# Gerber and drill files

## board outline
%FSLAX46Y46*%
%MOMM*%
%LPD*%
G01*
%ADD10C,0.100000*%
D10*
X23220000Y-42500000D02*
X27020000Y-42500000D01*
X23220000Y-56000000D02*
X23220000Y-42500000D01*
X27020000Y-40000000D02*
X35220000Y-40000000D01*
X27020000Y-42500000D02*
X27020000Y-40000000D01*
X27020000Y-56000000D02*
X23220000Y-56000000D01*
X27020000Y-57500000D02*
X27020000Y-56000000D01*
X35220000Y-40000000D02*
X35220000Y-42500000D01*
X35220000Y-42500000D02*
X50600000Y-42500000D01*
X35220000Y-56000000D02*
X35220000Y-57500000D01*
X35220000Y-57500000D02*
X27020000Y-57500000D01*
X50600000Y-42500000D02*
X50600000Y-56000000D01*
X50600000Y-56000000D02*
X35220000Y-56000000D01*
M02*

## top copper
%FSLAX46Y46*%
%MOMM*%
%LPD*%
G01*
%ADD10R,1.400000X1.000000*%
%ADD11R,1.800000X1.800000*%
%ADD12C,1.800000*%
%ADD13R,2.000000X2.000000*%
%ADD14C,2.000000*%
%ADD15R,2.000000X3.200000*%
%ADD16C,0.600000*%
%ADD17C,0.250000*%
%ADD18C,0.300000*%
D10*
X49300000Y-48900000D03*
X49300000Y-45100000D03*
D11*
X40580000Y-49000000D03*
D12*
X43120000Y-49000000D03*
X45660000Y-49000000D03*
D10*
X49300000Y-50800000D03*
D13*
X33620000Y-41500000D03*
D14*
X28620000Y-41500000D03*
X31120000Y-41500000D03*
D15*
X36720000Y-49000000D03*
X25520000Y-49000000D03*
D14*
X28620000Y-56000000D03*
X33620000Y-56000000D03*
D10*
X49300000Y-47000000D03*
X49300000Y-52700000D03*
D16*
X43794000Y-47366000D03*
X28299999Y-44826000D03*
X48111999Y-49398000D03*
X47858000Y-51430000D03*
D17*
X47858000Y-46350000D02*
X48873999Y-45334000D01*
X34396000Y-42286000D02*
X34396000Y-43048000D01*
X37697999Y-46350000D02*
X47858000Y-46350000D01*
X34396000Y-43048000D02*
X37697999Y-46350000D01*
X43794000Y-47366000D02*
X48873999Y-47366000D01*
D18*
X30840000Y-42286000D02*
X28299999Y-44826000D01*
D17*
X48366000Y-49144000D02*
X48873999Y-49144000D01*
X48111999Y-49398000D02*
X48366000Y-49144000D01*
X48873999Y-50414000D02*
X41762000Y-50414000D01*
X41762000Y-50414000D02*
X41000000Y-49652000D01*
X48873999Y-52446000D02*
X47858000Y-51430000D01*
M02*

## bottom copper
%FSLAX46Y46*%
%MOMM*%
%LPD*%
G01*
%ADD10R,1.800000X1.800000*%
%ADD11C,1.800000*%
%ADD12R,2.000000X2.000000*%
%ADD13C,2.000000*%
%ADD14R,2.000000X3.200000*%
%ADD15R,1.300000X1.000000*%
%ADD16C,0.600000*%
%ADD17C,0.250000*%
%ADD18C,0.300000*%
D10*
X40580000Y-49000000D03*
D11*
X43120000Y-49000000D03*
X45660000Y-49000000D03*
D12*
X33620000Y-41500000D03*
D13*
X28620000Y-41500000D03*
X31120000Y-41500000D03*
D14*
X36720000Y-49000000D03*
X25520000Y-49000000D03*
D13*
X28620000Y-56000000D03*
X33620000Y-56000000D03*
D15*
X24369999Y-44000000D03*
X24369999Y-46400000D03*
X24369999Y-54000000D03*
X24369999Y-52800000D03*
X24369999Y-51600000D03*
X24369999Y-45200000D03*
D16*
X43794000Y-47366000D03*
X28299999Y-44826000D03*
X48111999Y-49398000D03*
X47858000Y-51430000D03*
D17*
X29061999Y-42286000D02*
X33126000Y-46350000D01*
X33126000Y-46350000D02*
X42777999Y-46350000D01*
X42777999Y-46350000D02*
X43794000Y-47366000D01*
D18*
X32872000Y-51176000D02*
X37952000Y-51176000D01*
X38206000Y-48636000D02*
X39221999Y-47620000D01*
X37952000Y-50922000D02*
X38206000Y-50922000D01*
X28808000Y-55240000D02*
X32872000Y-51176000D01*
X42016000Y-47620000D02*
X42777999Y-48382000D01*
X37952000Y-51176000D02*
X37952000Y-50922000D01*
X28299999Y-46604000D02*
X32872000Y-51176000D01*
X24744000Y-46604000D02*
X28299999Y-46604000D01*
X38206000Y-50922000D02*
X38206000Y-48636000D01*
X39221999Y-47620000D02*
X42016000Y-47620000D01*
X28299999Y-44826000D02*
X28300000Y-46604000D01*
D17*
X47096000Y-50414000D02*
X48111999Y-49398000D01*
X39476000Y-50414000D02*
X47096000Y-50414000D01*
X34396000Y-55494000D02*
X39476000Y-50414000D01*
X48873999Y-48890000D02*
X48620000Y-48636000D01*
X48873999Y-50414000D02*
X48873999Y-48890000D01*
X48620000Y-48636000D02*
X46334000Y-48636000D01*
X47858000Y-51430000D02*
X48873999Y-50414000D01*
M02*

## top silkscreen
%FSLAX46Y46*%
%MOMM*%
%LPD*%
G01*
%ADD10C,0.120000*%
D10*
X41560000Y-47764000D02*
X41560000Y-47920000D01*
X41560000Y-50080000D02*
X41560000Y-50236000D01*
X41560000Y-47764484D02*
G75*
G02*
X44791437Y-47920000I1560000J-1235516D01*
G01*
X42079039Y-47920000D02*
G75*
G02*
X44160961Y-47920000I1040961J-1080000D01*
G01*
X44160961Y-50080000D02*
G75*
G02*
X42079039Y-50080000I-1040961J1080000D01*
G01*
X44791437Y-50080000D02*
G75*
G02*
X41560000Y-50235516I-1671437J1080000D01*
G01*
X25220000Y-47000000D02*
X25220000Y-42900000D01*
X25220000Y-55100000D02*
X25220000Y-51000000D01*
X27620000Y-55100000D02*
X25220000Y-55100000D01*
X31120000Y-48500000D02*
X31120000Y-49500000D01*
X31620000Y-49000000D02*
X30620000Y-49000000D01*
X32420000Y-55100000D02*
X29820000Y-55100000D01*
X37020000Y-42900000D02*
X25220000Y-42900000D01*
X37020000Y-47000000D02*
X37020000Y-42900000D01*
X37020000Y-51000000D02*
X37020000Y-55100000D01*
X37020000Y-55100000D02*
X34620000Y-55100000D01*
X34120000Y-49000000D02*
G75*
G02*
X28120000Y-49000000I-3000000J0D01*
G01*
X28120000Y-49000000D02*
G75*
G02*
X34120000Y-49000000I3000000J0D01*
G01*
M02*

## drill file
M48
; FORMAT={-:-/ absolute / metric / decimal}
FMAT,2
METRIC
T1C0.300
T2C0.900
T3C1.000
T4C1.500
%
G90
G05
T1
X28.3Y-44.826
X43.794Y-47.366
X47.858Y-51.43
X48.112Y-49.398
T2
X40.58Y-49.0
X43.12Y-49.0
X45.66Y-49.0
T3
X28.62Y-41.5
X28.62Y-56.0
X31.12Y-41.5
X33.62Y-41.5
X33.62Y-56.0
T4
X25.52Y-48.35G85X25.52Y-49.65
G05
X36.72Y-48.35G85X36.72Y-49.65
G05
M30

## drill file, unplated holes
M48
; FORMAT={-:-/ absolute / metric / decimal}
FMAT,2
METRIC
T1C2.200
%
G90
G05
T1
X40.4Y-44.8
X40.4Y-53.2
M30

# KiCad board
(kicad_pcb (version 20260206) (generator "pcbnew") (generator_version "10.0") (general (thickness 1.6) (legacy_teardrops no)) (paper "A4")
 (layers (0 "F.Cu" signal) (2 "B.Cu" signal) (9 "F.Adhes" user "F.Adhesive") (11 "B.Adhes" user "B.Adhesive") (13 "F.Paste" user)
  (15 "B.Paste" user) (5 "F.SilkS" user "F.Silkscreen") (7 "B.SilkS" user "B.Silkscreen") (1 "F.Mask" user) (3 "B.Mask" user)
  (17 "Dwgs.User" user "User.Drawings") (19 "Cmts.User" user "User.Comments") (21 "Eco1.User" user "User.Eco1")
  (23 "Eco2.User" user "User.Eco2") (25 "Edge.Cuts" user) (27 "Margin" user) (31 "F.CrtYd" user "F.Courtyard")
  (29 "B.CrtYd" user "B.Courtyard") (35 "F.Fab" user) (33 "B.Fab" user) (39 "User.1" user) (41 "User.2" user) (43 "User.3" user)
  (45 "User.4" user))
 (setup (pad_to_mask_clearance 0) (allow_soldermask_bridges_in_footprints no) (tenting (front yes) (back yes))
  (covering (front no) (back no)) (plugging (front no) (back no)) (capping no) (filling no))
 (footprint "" (layer "F.Cu") (at 49.3 48.9)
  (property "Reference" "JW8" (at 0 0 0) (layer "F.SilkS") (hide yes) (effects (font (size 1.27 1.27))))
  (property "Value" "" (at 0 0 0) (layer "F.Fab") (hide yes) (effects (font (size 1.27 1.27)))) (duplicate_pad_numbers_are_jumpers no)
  (pad "1" smd rect (at 0 0) (size 1.4 1) (layers "F.Cu" "F.Mask" "F.Paste") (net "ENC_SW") (thermal_bridge_angle 45)))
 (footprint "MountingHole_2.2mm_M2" (layer "F.Cu") (at 40.4 44.8)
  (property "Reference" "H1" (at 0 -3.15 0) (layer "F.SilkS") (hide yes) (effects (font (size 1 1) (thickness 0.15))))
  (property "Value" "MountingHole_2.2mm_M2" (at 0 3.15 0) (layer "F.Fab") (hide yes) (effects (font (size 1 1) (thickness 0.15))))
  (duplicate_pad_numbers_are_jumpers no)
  (pad "" np_thru_hole circle (at 0 0) (size 2.2 2.2) (drill 2.2) (layers "*.Cu" "*.Mask")))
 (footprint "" (layer "F.Cu") (at 49.3 45.1)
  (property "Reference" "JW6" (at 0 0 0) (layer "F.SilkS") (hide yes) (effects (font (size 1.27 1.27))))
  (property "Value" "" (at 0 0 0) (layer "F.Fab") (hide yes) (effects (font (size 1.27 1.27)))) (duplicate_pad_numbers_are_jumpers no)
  (pad "1" smd rect (at 0 0) (size 1.4 1) (layers "F.Cu" "F.Mask" "F.Paste") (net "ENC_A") (thermal_bridge_angle 45)))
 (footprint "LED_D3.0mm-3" (layer "F.Cu") (at 40.58 49)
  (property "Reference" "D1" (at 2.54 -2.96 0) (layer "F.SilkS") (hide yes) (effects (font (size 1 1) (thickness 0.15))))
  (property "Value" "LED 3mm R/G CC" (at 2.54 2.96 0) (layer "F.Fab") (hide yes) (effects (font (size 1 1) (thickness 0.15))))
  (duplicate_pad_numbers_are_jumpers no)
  (fp_line (start 0.98 -1.236) (end 0.98 -1.08) (stroke (width 0.12) (type solid)) (layer "F.SilkS"))
  (fp_line (start 0.98 1.08) (end 0.98 1.236) (stroke (width 0.12) (type solid)) (layer "F.SilkS"))
  (fp_arc (start 0.98 -1.235516) (mid 2.63566 -1.987699) (end 4.211437 -1.08) (stroke (width 0.12) (type solid)) (layer "F.SilkS"))
  (fp_arc (start 1.499039 -1.08) (mid 2.54 -1.5) (end 3.580961 -1.08) (stroke (width 0.12) (type solid)) (layer "F.SilkS"))
  (fp_arc (start 3.580961 1.08) (mid 2.54 1.5) (end 1.499039 1.08) (stroke (width 0.12) (type solid)) (layer "F.SilkS"))
  (fp_arc (start 4.211437 1.08) (mid 2.63566 1.987699) (end 0.98 1.235516) (stroke (width 0.12) (type solid)) (layer "F.SilkS"))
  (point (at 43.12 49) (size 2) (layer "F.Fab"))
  (pad "1" thru_hole rect (at 0 0) (size 1.8 1.8) (drill 0.9) (layers "*.Cu" "*.Mask") (remove_unused_layers no) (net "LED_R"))
  (pad "2" thru_hole circle (at 2.54 0) (size 1.8 1.8) (drill 0.9) (layers "*.Cu" "*.Mask") (remove_unused_layers no) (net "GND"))
  (pad "3" thru_hole circle (at 5.08 0) (size 1.8 1.8) (drill 0.9) (layers "*.Cu" "*.Mask") (remove_unused_layers no) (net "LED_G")))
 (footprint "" (layer "F.Cu") (at 49.3 50.8)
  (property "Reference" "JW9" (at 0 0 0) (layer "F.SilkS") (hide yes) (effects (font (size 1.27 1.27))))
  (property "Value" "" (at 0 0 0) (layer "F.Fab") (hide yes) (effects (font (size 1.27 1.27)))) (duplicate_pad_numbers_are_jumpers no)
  (pad "1" smd rect (at 0 0) (size 1.4 1) (layers "F.Cu" "F.Mask" "F.Paste") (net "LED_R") (thermal_bridge_angle 45)))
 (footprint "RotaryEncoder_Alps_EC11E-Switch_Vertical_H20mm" (layer "F.Cu") (at 33.62 41.5 -90)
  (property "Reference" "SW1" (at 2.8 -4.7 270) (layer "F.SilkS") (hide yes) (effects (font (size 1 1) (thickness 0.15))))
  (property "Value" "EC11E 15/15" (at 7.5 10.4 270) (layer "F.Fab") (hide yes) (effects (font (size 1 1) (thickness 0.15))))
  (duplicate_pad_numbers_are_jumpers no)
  (fp_line (start 5.5 8.4) (end 1.4 8.4) (stroke (width 0.12) (type solid)) (layer "F.SilkS"))
  (fp_line (start 13.6 8.4) (end 9.5 8.4) (stroke (width 0.12) (type solid)) (layer "F.SilkS"))
  (fp_line (start 13.6 6) (end 13.6 8.4) (stroke (width 0.12) (type solid)) (layer "F.SilkS"))
  (fp_line (start 7 2.5) (end 8 2.5) (stroke (width 0.12) (type solid)) (layer "F.SilkS"))
  (fp_line (start 7.5 2) (end 7.5 3) (stroke (width 0.12) (type solid)) (layer "F.SilkS"))
  (fp_line (start 13.6 1.2) (end 13.6 3.8) (stroke (width 0.12) (type solid)) (layer "F.SilkS"))
  (fp_line (start 1.4 -3.4) (end 1.4 8.4) (stroke (width 0.12) (type solid)) (layer "F.SilkS"))
  (fp_line (start 5.5 -3.4) (end 1.4 -3.4) (stroke (width 0.12) (type solid)) (layer "F.SilkS"))
  (fp_line (start 9.5 -3.4) (end 13.6 -3.4) (stroke (width 0.12) (type solid)) (layer "F.SilkS"))
  (fp_line (start 13.6 -3.4) (end 13.6 -1) (stroke (width 0.12) (type solid)) (layer "F.SilkS"))
  (fp_circle (center 7.5 2.5) (end 10.5 2.5) (stroke (width 0.12) (type solid)) (fill no) (layer "F.SilkS"))
  (pad "A" thru_hole rect (at 0 0 270) (size 2 2) (drill 1) (layers "*.Cu" "*.Mask") (remove_unused_layers no) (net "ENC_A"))
  (pad "B" thru_hole circle (at 0 5 270) (size 2 2) (drill 1) (layers "*.Cu" "*.Mask") (remove_unused_layers no) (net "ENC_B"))
  (pad "C" thru_hole circle (at 0 2.5 270) (size 2 2) (drill 1) (layers "*.Cu" "*.Mask") (remove_unused_layers no) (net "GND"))
  (pad "MP" thru_hole rect (at 7.5 -3.1 270) (size 3.2 2) (drill oval 2.8 1.5) (layers "*.Cu" "*.Mask") (remove_unused_layers no))
  (pad "MP" thru_hole rect (at 7.5 8.1 270) (size 3.2 2) (drill oval 2.8 1.5) (layers "*.Cu" "*.Mask") (remove_unused_layers no))
  (pad "S1" thru_hole circle (at 14.5 5 270) (size 2 2) (drill 1) (layers "*.Cu" "*.Mask") (remove_unused_layers no) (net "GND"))
  (pad "S2" thru_hole circle (at 14.5 0 270) (size 2 2) (drill 1) (layers "*.Cu" "*.Mask") (remove_unused_layers no) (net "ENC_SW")))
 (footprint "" (layer "F.Cu") (at 49.3 47)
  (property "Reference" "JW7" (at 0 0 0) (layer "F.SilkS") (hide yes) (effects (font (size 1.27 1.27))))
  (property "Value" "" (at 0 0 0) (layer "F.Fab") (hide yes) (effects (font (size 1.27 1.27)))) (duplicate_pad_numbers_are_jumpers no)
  (pad "1" smd rect (at 0 0) (size 1.4 1) (layers "F.Cu" "F.Mask" "F.Paste") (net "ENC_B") (thermal_bridge_angle 45)))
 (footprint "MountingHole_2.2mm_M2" (layer "F.Cu") (at 40.4 53.2)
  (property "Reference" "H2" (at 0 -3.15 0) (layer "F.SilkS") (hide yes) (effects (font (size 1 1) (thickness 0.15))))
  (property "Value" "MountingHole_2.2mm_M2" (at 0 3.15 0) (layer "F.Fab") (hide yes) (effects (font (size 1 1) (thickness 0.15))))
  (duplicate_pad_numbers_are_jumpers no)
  (pad "" np_thru_hole circle (at 0 0) (size 2.2 2.2) (drill 2.2) (layers "*.Cu" "*.Mask")))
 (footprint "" (layer "F.Cu") (at 49.3 52.7)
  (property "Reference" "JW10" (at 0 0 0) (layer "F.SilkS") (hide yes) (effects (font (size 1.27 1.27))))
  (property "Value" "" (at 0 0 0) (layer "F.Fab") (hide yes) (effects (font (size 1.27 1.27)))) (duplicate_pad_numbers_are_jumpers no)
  (pad "1" smd rect (at 0 0) (size 1.4 1) (layers "F.Cu" "F.Mask" "F.Paste") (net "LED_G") (thermal_bridge_angle 45)))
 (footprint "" (layer "B.Cu") (at 24.369999 44 180)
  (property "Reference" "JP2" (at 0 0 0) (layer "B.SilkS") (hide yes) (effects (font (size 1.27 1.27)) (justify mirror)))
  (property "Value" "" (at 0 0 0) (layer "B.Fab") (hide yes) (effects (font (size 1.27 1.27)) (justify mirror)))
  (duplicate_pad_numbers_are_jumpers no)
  (pad "1" smd rect (at 0 0 180) (size 1.3 1) (layers "B.Cu" "B.Mask" "B.Paste") (thermal_bridge_angle 45)))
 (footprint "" (layer "B.Cu") (at 24.369999 46.4 180)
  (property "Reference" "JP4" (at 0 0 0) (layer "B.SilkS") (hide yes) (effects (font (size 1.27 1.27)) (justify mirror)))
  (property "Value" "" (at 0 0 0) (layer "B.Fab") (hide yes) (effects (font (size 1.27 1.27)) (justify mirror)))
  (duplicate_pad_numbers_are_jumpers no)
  (pad "1" smd rect (at 0 0 180) (size 1.3 1) (layers "B.Cu" "B.Mask" "B.Paste") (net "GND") (thermal_bridge_angle 45)))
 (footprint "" (layer "B.Cu") (at 24.369999 54 180)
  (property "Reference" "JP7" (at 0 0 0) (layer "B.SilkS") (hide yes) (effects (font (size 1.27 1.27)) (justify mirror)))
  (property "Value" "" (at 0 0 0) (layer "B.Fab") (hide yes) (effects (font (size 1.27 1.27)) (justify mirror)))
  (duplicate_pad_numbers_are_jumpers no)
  (pad "1" smd rect (at 0 0 180) (size 1.3 1) (layers "B.Cu" "B.Mask" "B.Paste") (thermal_bridge_angle 45)))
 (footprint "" (layer "B.Cu") (at 24.369999 52.8 180)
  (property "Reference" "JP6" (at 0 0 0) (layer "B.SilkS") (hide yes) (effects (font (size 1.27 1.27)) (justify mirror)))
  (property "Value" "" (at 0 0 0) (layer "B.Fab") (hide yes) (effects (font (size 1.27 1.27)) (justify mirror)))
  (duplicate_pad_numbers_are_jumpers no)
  (pad "1" smd rect (at 0 0 180) (size 1.3 1) (layers "B.Cu" "B.Mask" "B.Paste") (thermal_bridge_angle 45)))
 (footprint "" (layer "B.Cu") (at 24.369999 51.6 180)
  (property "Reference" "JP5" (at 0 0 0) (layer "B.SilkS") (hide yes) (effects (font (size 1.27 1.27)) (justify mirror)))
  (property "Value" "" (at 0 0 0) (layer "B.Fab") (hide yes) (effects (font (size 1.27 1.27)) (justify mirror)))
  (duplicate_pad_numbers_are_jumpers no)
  (pad "1" smd rect (at 0 0 180) (size 1.3 1) (layers "B.Cu" "B.Mask" "B.Paste") (thermal_bridge_angle 45)))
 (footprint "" (layer "B.Cu") (at 24.369999 45.2 180)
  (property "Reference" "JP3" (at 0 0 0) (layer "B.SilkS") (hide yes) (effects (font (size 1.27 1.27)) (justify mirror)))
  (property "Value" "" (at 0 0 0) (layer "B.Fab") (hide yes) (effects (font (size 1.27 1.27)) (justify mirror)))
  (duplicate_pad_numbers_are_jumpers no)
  (pad "1" smd rect (at 0 0 180) (size 1.3 1) (layers "B.Cu" "B.Mask" "B.Paste") (thermal_bridge_angle 45)))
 (gr_line (start 23.22 42.5) (end 27.02 42.5) (stroke (width 0.1) (type default)) (layer "Edge.Cuts"))
 (gr_line (start 23.22 56) (end 23.22 42.5) (stroke (width 0.1) (type default)) (layer "Edge.Cuts"))
 (gr_line (start 27.02 40) (end 35.22 40) (stroke (width 0.1) (type default)) (layer "Edge.Cuts"))
 (gr_line (start 27.02 42.5) (end 27.02 40) (stroke (width 0.1) (type default)) (layer "Edge.Cuts"))
 (gr_line (start 27.02 56) (end 23.22 56) (stroke (width 0.1) (type default)) (layer "Edge.Cuts"))
 (gr_line (start 27.02 57.5) (end 27.02 56) (stroke (width 0.1) (type default)) (layer "Edge.Cuts"))
 (gr_line (start 35.22 40) (end 35.22 42.5) (stroke (width 0.1) (type default)) (layer "Edge.Cuts"))
 (gr_line (start 35.22 42.5) (end 50.6 42.5) (stroke (width 0.1) (type default)) (layer "Edge.Cuts"))
 (gr_line (start 35.22 56) (end 35.22 57.5) (stroke (width 0.1) (type default)) (layer "Edge.Cuts"))
 (gr_line (start 35.22 57.5) (end 27.02 57.5) (stroke (width 0.1) (type default)) (layer "Edge.Cuts"))
 (gr_line (start 50.6 42.5) (end 50.6 56) (stroke (width 0.1) (type default)) (layer "Edge.Cuts"))
 (gr_line (start 50.6 56) (end 35.22 56) (stroke (width 0.1) (type default)) (layer "Edge.Cuts"))
 (segment (start 47.858 46.35) (end 48.873999 45.334) (width 0.25) (layer "F.Cu") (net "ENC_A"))
 (segment (start 34.396 42.286) (end 34.396 43.048) (width 0.25) (layer "F.Cu") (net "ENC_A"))
 (segment (start 37.697999 46.35) (end 47.858 46.35) (width 0.25) (layer "F.Cu") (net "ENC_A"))
 (segment (start 34.396 43.048) (end 37.697999 46.35) (width 0.25) (layer "F.Cu") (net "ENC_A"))
 (segment (start 43.794 47.366) (end 48.873999 47.366) (width 0.25) (layer "F.Cu") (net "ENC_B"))
 (via (at 43.794 47.366) (size 0.6) (drill 0.3) (layers "F.Cu" "B.Cu") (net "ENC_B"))
 (segment (start 29.061999 42.286) (end 33.126 46.35) (width 0.25) (layer "B.Cu") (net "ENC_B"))
 (segment (start 33.126 46.35) (end 42.777999 46.35) (width 0.25) (layer "B.Cu") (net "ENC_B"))
 (segment (start 42.777999 46.35) (end 43.794 47.366) (width 0.25) (layer "B.Cu") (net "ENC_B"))
 (segment (start 30.84 42.286) (end 28.299999 44.826) (width 0.3) (layer "F.Cu") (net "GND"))
 (via (at 28.299999 44.826) (size 0.6) (drill 0.3) (layers "F.Cu" "B.Cu") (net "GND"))
 (segment (start 32.872 51.176) (end 37.952 51.176) (width 0.3) (layer "B.Cu") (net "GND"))
 (segment (start 38.206 48.636) (end 39.221999 47.62) (width 0.3) (layer "B.Cu") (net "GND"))
 (segment (start 37.952 50.922) (end 38.206 50.922) (width 0.3) (layer "B.Cu") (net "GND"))
 (segment (start 28.808 55.24) (end 32.872 51.176) (width 0.3) (layer "B.Cu") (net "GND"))
 (segment (start 42.016 47.62) (end 42.777999 48.382) (width 0.3) (layer "B.Cu") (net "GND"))
 (segment (start 37.952 51.176) (end 37.952 50.922) (width 0.3) (layer "B.Cu") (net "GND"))
 (segment (start 28.299999 46.604) (end 32.872 51.176) (width 0.3) (layer "B.Cu") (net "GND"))
 (segment (start 24.744 46.604) (end 28.299999 46.604) (width 0.3) (layer "B.Cu") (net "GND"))
 (segment (start 38.206 50.922) (end 38.206 48.636) (width 0.3) (layer "B.Cu") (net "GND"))
 (segment (start 39.221999 47.62) (end 42.016 47.62) (width 0.3) (layer "B.Cu") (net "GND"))
 (segment (start 28.299999 44.826) (end 28.3 46.604) (width 0.3) (layer "B.Cu") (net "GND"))
 (segment (start 48.366 49.144) (end 48.873999 49.144) (width 0.25) (layer "F.Cu") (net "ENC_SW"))
 (segment (start 48.111999 49.398) (end 48.366 49.144) (width 0.25) (layer "F.Cu") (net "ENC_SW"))
 (via (at 48.111999 49.398) (size 0.6) (drill 0.3) (layers "F.Cu" "B.Cu") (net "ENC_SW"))
 (segment (start 47.096 50.414) (end 48.111999 49.398) (width 0.25) (layer "B.Cu") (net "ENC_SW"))
 (segment (start 39.476 50.414) (end 47.096 50.414) (width 0.25) (layer "B.Cu") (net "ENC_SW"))
 (segment (start 34.396 55.494) (end 39.476 50.414) (width 0.25) (layer "B.Cu") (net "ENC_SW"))
 (segment (start 48.873999 50.414) (end 41.762 50.414) (width 0.25) (layer "F.Cu") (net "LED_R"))
 (segment (start 41.762 50.414) (end 41 49.652) (width 0.25) (layer "F.Cu") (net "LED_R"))
 (segment (start 48.873999 52.446) (end 47.858 51.43) (width 0.25) (layer "F.Cu") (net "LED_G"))
 (via (at 47.858 51.43) (size 0.6) (drill 0.3) (layers "F.Cu" "B.Cu") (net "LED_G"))
 (segment (start 48.873999 48.89) (end 48.62 48.636) (width 0.25) (layer "B.Cu") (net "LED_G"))
 (segment (start 48.873999 50.414) (end 48.873999 48.89) (width 0.25) (layer "B.Cu") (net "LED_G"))
 (segment (start 48.62 48.636) (end 46.334 48.636) (width 0.25) (layer "B.Cu") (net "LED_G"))
 (segment (start 47.858 51.43) (end 48.873999 50.414) (width 0.25) (layer "B.Cu") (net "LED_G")))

